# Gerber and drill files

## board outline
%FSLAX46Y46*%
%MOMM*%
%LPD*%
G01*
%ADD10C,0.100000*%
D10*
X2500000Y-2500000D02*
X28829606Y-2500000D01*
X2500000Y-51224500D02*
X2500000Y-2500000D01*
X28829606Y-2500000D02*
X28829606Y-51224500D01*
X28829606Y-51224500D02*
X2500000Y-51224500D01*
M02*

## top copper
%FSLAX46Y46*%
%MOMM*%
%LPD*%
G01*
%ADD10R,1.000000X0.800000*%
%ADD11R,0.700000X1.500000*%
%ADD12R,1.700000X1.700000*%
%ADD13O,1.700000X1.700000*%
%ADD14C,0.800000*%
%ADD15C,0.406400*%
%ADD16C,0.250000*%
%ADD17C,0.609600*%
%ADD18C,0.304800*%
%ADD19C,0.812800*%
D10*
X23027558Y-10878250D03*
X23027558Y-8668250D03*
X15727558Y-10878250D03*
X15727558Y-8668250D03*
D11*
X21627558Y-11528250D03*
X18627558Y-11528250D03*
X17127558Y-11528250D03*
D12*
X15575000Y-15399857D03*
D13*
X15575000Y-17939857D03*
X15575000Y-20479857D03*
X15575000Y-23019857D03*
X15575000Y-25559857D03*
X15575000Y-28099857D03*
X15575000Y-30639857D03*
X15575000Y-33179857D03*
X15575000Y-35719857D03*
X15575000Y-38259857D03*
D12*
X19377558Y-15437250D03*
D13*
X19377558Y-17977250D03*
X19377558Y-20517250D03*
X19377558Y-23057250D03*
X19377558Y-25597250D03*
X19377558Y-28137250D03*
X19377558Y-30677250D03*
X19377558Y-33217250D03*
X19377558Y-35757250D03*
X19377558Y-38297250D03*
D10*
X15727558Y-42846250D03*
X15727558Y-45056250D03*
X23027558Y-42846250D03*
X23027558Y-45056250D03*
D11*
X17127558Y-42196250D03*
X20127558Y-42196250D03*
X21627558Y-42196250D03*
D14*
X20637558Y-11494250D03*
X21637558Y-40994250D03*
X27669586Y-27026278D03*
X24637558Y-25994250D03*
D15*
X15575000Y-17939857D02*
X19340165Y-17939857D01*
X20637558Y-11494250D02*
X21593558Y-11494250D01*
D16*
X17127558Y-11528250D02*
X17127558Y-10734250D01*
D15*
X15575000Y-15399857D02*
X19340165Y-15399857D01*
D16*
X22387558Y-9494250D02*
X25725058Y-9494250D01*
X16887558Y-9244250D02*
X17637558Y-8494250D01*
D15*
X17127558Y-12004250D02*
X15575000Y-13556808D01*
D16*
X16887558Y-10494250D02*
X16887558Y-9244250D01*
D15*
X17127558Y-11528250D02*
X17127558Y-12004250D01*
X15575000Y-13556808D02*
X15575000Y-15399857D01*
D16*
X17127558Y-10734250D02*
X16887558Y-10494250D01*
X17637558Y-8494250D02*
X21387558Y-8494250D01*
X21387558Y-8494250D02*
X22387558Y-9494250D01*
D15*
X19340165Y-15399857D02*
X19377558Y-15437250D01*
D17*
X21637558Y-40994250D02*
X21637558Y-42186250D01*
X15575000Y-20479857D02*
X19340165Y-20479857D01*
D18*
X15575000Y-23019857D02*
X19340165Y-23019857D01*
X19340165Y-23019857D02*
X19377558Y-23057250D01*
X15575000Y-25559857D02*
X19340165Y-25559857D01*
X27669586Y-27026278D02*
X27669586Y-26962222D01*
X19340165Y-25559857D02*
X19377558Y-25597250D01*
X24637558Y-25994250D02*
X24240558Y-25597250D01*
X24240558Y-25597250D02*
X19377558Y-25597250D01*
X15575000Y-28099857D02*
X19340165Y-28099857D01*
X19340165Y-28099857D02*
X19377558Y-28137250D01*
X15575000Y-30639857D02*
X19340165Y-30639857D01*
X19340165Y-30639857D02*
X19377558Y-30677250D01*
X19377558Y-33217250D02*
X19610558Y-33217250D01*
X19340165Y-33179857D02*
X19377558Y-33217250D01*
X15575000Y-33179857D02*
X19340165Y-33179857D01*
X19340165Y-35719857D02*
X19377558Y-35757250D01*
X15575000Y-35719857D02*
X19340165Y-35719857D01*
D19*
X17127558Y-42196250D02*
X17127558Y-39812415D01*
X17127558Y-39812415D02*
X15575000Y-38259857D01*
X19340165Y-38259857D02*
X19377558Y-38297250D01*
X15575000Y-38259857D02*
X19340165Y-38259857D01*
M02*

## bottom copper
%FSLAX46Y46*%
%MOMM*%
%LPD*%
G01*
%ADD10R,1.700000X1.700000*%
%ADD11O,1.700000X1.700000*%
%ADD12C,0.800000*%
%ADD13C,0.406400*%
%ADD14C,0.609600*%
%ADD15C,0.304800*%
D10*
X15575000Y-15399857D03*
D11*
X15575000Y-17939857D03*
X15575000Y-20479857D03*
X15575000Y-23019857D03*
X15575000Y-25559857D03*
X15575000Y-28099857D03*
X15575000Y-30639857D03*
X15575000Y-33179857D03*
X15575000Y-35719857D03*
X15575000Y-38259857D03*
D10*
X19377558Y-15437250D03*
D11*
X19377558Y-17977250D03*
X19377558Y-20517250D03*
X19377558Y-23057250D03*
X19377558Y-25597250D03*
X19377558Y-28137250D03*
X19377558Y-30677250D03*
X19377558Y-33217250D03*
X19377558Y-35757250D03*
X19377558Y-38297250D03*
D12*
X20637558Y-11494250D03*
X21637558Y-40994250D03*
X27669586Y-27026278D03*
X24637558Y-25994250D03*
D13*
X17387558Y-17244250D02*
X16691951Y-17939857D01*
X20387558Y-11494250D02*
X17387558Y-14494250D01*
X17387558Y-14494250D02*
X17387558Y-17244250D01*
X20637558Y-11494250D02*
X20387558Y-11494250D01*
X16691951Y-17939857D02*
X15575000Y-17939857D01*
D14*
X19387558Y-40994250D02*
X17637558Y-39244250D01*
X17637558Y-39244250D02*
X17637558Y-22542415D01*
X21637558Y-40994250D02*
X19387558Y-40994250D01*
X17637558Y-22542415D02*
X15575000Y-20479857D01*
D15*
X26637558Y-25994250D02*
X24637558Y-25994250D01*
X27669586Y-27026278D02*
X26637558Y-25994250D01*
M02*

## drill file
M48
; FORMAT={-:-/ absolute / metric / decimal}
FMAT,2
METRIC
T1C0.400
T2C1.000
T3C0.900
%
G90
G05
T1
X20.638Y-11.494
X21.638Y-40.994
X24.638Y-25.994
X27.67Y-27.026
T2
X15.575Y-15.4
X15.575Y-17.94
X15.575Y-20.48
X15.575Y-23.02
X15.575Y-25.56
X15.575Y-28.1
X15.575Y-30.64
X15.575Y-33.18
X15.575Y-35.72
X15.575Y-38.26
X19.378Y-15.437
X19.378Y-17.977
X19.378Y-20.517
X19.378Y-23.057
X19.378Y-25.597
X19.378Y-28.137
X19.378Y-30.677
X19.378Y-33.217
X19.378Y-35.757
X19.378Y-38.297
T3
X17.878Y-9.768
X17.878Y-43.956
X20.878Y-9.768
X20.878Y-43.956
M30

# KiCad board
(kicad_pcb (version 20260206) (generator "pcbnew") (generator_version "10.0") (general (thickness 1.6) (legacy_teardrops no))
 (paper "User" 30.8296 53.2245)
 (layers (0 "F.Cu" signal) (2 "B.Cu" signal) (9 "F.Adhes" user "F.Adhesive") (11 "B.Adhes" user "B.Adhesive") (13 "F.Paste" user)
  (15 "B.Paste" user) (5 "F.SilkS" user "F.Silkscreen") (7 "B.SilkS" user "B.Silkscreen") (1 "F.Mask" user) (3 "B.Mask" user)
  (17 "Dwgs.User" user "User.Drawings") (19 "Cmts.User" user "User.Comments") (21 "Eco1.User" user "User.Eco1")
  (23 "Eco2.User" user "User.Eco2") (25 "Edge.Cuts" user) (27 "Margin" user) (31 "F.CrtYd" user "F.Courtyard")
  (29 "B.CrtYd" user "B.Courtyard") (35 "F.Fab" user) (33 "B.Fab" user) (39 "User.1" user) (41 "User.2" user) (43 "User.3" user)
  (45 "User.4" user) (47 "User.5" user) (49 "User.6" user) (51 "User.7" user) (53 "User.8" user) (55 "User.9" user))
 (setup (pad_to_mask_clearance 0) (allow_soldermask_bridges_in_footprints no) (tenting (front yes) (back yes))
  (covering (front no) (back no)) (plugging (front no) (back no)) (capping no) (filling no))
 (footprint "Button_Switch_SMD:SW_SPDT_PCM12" (layer "F.Cu") (at 19.377558 10.09825 180)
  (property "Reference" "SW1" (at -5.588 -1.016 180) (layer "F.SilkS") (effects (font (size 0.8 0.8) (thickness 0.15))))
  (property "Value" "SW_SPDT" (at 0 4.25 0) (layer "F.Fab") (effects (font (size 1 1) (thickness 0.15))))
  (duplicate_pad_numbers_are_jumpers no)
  (pad "" smd rect (at -3.65 -0.78 180) (size 1 0.8) (layers "F.Cu" "F.Mask" "F.Paste"))
  (pad "" smd rect (at -3.65 1.43 180) (size 1 0.8) (layers "F.Cu" "F.Mask" "F.Paste"))
  (pad "" np_thru_hole circle (at -1.5 0.33 180) (size 0.9 0.9) (drill 0.9) (layers "*.Cu" "*.Mask"))
  (pad "" np_thru_hole circle (at 1.5 0.33 180) (size 0.9 0.9) (drill 0.9) (layers "*.Cu" "*.Mask"))
  (pad "" smd rect (at 3.65 -0.78 180) (size 1 0.8) (layers "F.Cu" "F.Mask" "F.Paste"))
  (pad "" smd rect (at 3.65 1.43 180) (size 1 0.8) (layers "F.Cu" "F.Mask" "F.Paste"))
  (pad "1" smd rect (at -2.25 -1.43 180) (size 0.7 1.5) (layers "F.Cu" "F.Mask" "F.Paste") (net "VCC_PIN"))
  (pad "2" smd rect (at 0.75 -1.43 180) (size 0.7 1.5) (layers "F.Cu" "F.Mask" "F.Paste") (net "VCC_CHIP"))
  (pad "3" smd rect (at 2.25 -1.43 180) (size 0.7 1.5) (layers "F.Cu" "F.Mask" "F.Paste") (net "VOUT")))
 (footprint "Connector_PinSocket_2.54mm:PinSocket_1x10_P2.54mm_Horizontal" (layer "F.Cu") (at 15.575 15.399857)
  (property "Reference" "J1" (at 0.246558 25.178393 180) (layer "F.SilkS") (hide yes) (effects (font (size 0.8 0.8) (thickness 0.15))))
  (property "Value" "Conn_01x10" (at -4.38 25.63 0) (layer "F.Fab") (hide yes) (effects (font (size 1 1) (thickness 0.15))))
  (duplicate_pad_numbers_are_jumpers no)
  (pad "1" thru_hole rect (at 0 0) (size 1.7 1.7) (drill 1) (layers "*.Cu" "*.Mask") (remove_unused_layers no) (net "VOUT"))
  (pad "2" thru_hole oval (at 0 2.54) (size 1.7 1.7) (drill 1) (layers "*.Cu" "*.Mask") (remove_unused_layers no) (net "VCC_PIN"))
  (pad "3" thru_hole oval (at 0 5.08) (size 1.7 1.7) (drill 1) (layers "*.Cu" "*.Mask") (remove_unused_layers no) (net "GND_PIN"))
  (pad "4" thru_hole oval (at 0 7.62) (size 1.7 1.7) (drill 1) (layers "*.Cu" "*.Mask") (remove_unused_layers no) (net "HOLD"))
  (pad "5" thru_hole oval (at 0 10.16) (size 1.7 1.7) (drill 1) (layers "*.Cu" "*.Mask") (remove_unused_layers no) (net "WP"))
  (pad "6" thru_hole oval (at 0 12.7) (size 1.7 1.7) (drill 1) (layers "*.Cu" "*.Mask") (remove_unused_layers no) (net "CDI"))
  (pad "7" thru_hole oval (at 0 15.24) (size 1.7 1.7) (drill 1) (layers "*.Cu" "*.Mask") (remove_unused_layers no) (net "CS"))
  (pad "8" thru_hole oval (at 0 17.78) (size 1.7 1.7) (drill 1) (layers "*.Cu" "*.Mask") (remove_unused_layers no) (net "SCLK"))
  (pad "9" thru_hole oval (at 0 20.32) (size 1.7 1.7) (drill 1) (layers "*.Cu" "*.Mask") (remove_unused_layers no) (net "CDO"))
  (pad "10" thru_hole oval (at 0 22.86) (size 1.7 1.7) (drill 1) (layers "*.Cu" "*.Mask") (remove_unused_layers no) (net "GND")))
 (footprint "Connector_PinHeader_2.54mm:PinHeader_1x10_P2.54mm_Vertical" (layer "F.Cu") (at 19.377558 15.43725)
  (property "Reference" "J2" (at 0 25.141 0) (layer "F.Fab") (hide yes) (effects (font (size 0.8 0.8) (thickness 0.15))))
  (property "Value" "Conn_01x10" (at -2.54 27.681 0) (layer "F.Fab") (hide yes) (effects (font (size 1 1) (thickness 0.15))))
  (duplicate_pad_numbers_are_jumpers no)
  (pad "1" thru_hole rect (at 0 0) (size 1.7 1.7) (drill 1) (layers "*.Cu" "*.Mask") (remove_unused_layers no) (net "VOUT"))
  (pad "2" thru_hole oval (at 0 2.54) (size 1.7 1.7) (drill 1) (layers "*.Cu" "*.Mask") (remove_unused_layers no) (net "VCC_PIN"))
  (pad "3" thru_hole oval (at 0 5.08) (size 1.7 1.7) (drill 1) (layers "*.Cu" "*.Mask") (remove_unused_layers no) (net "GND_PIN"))
  (pad "4" thru_hole oval (at 0 7.62) (size 1.7 1.7) (drill 1) (layers "*.Cu" "*.Mask") (remove_unused_layers no) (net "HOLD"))
  (pad "5" thru_hole oval (at 0 10.16) (size 1.7 1.7) (drill 1) (layers "*.Cu" "*.Mask") (remove_unused_layers no) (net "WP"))
  (pad "6" thru_hole oval (at 0 12.7) (size 1.7 1.7) (drill 1) (layers "*.Cu" "*.Mask") (remove_unused_layers no) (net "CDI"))
  (pad "7" thru_hole oval (at 0 15.24) (size 1.7 1.7) (drill 1) (layers "*.Cu" "*.Mask") (remove_unused_layers no) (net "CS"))
  (pad "8" thru_hole oval (at 0 17.78) (size 1.7 1.7) (drill 1) (layers "*.Cu" "*.Mask") (remove_unused_layers no) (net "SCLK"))
  (pad "9" thru_hole oval (at 0 20.32) (size 1.7 1.7) (drill 1) (layers "*.Cu" "*.Mask") (remove_unused_layers no) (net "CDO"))
  (pad "10" thru_hole oval (at 0 22.86) (size 1.7 1.7) (drill 1) (layers "*.Cu" "*.Mask") (remove_unused_layers no) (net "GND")))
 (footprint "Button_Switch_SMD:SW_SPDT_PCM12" (layer "F.Cu") (at 19.377558 43.62625)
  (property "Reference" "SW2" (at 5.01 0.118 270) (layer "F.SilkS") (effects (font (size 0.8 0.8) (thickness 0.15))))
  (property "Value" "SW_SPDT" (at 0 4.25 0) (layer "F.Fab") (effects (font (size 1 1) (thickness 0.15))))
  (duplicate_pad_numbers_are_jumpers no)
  (pad "" smd rect (at -3.65 -0.78) (size 1 0.8) (layers "F.Cu" "F.Mask" "F.Paste"))
  (pad "" smd rect (at -3.65 1.43) (size 1 0.8) (layers "F.Cu" "F.Mask" "F.Paste"))
  (pad "" np_thru_hole circle (at -1.5 0.33) (size 0.9 0.9) (drill 0.9) (layers "*.Cu" "*.Mask"))
  (pad "" np_thru_hole circle (at 1.5 0.33) (size 0.9 0.9) (drill 0.9) (layers "*.Cu" "*.Mask"))
  (pad "" smd rect (at 3.65 -0.78) (size 1 0.8) (layers "F.Cu" "F.Mask" "F.Paste"))
  (pad "" smd rect (at 3.65 1.43) (size 1 0.8) (layers "F.Cu" "F.Mask" "F.Paste"))
  (pad "1" smd rect (at -2.25 -1.43) (size 0.7 1.5) (layers "F.Cu" "F.Mask" "F.Paste") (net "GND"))
  (pad "2" smd rect (at 0.75 -1.43) (size 0.7 1.5) (layers "F.Cu" "F.Mask" "F.Paste") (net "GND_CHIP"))
  (pad "3" smd rect (at 2.25 -1.43) (size 0.7 1.5) (layers "F.Cu" "F.Mask" "F.Paste") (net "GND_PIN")))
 (gr_line (start 2.5 2.5) (end 28.829606 2.5) (stroke (width 0.1) (type default)) (layer "Edge.Cuts"))
 (gr_line (start 2.5 51.2245) (end 2.5 2.5) (stroke (width 0.1) (type default)) (layer "Edge.Cuts"))
 (gr_line (start 28.829606 2.5) (end 28.829606 51.2245) (stroke (width 0.1) (type default)) (layer "Edge.Cuts"))
 (gr_line (start 28.829606 51.2245) (end 2.5 51.2245) (stroke (width 0.1) (type default)) (layer "Edge.Cuts"))
 (segment (start 15.575 17.939857) (end 19.340165 17.939857) (width 0.4064) (layer "F.Cu") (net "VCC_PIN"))
 (segment (start 20.637558 11.49425) (end 21.593558 11.49425) (width 0.4064) (layer "F.Cu") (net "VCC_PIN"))
 (via (at 20.637558 11.49425) (size 0.8) (drill 0.4) (layers "F.Cu" "B.Cu") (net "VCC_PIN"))
 (segment (start 17.387558 17.24425) (end 16.691951 17.939857) (width 0.4064) (layer "B.Cu") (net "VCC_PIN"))
 (segment (start 20.387558 11.49425) (end 17.387558 14.49425) (width 0.4064) (layer "B.Cu") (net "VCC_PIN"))
 (segment (start 17.387558 14.49425) (end 17.387558 17.24425) (width 0.4064) (layer "B.Cu") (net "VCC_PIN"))
 (segment (start 20.637558 11.49425) (end 20.387558 11.49425) (width 0.4064) (layer "B.Cu") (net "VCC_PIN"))
 (segment (start 16.691951 17.939857) (end 15.575 17.939857) (width 0.4064) (layer "B.Cu") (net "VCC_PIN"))
 (segment (start 17.127558 11.52825) (end 17.127558 10.73425) (width 0.25) (layer "F.Cu") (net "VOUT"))
 (segment (start 15.575 15.399857) (end 19.340165 15.399857) (width 0.4064) (layer "F.Cu") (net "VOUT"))
 (segment (start 22.387558 9.49425) (end 25.725058 9.49425) (width 0.25) (layer "F.Cu") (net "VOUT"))
 (segment (start 16.887558 9.24425) (end 17.637558 8.49425) (width 0.25) (layer "F.Cu") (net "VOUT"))
 (segment (start 17.127558 12.00425) (end 15.575 13.556808) (width 0.4064) (layer "F.Cu") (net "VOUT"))
 (segment (start 16.887558 10.49425) (end 16.887558 9.24425) (width 0.25) (layer "F.Cu") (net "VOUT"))
 (segment (start 17.127558 11.52825) (end 17.127558 12.00425) (width 0.4064) (layer "F.Cu") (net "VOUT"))
 (segment (start 15.575 13.556808) (end 15.575 15.399857) (width 0.4064) (layer "F.Cu") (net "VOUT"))
 (segment (start 17.127558 10.73425) (end 16.887558 10.49425) (width 0.25) (layer "F.Cu") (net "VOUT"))
 (segment (start 17.637558 8.49425) (end 21.387558 8.49425) (width 0.25) (layer "F.Cu") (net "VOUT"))
 (segment (start 21.387558 8.49425) (end 22.387558 9.49425) (width 0.25) (layer "F.Cu") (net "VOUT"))
 (segment (start 19.340165 15.399857) (end 19.377558 15.43725) (width 0.4064) (layer "F.Cu") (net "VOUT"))
 (segment (start 21.637558 40.99425) (end 21.637558 42.18625) (width 0.6096) (layer "F.Cu") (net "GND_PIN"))
 (segment (start 15.575 20.479857) (end 19.340165 20.479857) (width 0.6096) (layer "F.Cu") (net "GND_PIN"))
 (via (at 21.637558 40.99425) (size 0.8) (drill 0.4) (layers "F.Cu" "B.Cu") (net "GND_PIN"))
 (segment (start 19.387558 40.99425) (end 17.637558 39.24425) (width 0.6096) (layer "B.Cu") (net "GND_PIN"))
 (segment (start 17.637558 39.24425) (end 17.637558 22.542415) (width 0.6096) (layer "B.Cu") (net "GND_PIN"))
 (segment (start 21.637558 40.99425) (end 19.387558 40.99425) (width 0.6096) (layer "B.Cu") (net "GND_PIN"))
 (segment (start 17.637558 22.542415) (end 15.575 20.479857) (width 0.6096) (layer "B.Cu") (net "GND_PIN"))
 (segment (start 15.575 23.019857) (end 19.340165 23.019857) (width 0.3048) (layer "F.Cu") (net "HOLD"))
 (segment (start 19.340165 23.019857) (end 19.377558 23.05725) (width 0.3048) (layer "F.Cu") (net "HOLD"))
 (segment (start 15.575 25.559857) (end 19.340165 25.559857) (width 0.3048) (layer "F.Cu") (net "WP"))
 (segment (start 27.669586 27.026278) (end 27.669586 26.962222) (width 0.3048) (layer "F.Cu") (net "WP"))
 (segment (start 19.340165 25.559857) (end 19.377558 25.59725) (width 0.3048) (layer "F.Cu") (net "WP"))
 (segment (start 24.637558 25.99425) (end 24.240558 25.59725) (width 0.3048) (layer "F.Cu") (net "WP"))
 (segment (start 24.240558 25.59725) (end 19.377558 25.59725) (width 0.3048) (layer "F.Cu") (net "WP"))
 (via (at 27.669586 27.026278) (size 0.8) (drill 0.4) (layers "F.Cu" "B.Cu") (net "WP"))
 (via (at 24.637558 25.99425) (size 0.8) (drill 0.4) (layers "F.Cu" "B.Cu") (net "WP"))
 (segment (start 26.637558 25.99425) (end 24.637558 25.99425) (width 0.3048) (layer "B.Cu") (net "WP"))
 (segment (start 27.669586 27.026278) (end 26.637558 25.99425) (width 0.3048) (layer "B.Cu") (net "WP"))
 (segment (start 15.575 28.099857) (end 19.340165 28.099857) (width 0.3048) (layer "F.Cu") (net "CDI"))
 (segment (start 19.340165 28.099857) (end 19.377558 28.13725) (width 0.3048) (layer "F.Cu") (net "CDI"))
 (segment (start 15.575 30.639857) (end 19.340165 30.639857) (width 0.3048) (layer "F.Cu") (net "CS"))
 (segment (start 19.340165 30.639857) (end 19.377558 30.67725) (width 0.3048) (layer "F.Cu") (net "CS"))
 (segment (start 19.377558 33.21725) (end 19.610558 33.21725) (width 0.3048) (layer "F.Cu") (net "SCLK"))
 (segment (start 19.340165 33.179857) (end 19.377558 33.21725) (width 0.3048) (layer "F.Cu") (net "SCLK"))
 (segment (start 15.575 33.179857) (end 19.340165 33.179857) (width 0.3048) (layer "F.Cu") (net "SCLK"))
 (segment (start 19.340165 35.719857) (end 19.377558 35.75725) (width 0.3048) (layer "F.Cu") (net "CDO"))
 (segment (start 15.575 35.719857) (end 19.340165 35.719857) (width 0.3048) (layer "F.Cu") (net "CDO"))
 (segment (start 17.127558 42.19625) (end 17.127558 39.812415) (width 0.8128) (layer "F.Cu") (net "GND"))
 (segment (start 17.127558 39.812415) (end 15.575 38.259857) (width 0.8128) (layer "F.Cu") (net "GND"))
 (segment (start 19.340165 38.259857) (end 19.377558 38.29725) (width 0.8128) (layer "F.Cu") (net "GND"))
 (segment (start 15.575 38.259857) (end 19.340165 38.259857) (width 0.8128) (layer "F.Cu") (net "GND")))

